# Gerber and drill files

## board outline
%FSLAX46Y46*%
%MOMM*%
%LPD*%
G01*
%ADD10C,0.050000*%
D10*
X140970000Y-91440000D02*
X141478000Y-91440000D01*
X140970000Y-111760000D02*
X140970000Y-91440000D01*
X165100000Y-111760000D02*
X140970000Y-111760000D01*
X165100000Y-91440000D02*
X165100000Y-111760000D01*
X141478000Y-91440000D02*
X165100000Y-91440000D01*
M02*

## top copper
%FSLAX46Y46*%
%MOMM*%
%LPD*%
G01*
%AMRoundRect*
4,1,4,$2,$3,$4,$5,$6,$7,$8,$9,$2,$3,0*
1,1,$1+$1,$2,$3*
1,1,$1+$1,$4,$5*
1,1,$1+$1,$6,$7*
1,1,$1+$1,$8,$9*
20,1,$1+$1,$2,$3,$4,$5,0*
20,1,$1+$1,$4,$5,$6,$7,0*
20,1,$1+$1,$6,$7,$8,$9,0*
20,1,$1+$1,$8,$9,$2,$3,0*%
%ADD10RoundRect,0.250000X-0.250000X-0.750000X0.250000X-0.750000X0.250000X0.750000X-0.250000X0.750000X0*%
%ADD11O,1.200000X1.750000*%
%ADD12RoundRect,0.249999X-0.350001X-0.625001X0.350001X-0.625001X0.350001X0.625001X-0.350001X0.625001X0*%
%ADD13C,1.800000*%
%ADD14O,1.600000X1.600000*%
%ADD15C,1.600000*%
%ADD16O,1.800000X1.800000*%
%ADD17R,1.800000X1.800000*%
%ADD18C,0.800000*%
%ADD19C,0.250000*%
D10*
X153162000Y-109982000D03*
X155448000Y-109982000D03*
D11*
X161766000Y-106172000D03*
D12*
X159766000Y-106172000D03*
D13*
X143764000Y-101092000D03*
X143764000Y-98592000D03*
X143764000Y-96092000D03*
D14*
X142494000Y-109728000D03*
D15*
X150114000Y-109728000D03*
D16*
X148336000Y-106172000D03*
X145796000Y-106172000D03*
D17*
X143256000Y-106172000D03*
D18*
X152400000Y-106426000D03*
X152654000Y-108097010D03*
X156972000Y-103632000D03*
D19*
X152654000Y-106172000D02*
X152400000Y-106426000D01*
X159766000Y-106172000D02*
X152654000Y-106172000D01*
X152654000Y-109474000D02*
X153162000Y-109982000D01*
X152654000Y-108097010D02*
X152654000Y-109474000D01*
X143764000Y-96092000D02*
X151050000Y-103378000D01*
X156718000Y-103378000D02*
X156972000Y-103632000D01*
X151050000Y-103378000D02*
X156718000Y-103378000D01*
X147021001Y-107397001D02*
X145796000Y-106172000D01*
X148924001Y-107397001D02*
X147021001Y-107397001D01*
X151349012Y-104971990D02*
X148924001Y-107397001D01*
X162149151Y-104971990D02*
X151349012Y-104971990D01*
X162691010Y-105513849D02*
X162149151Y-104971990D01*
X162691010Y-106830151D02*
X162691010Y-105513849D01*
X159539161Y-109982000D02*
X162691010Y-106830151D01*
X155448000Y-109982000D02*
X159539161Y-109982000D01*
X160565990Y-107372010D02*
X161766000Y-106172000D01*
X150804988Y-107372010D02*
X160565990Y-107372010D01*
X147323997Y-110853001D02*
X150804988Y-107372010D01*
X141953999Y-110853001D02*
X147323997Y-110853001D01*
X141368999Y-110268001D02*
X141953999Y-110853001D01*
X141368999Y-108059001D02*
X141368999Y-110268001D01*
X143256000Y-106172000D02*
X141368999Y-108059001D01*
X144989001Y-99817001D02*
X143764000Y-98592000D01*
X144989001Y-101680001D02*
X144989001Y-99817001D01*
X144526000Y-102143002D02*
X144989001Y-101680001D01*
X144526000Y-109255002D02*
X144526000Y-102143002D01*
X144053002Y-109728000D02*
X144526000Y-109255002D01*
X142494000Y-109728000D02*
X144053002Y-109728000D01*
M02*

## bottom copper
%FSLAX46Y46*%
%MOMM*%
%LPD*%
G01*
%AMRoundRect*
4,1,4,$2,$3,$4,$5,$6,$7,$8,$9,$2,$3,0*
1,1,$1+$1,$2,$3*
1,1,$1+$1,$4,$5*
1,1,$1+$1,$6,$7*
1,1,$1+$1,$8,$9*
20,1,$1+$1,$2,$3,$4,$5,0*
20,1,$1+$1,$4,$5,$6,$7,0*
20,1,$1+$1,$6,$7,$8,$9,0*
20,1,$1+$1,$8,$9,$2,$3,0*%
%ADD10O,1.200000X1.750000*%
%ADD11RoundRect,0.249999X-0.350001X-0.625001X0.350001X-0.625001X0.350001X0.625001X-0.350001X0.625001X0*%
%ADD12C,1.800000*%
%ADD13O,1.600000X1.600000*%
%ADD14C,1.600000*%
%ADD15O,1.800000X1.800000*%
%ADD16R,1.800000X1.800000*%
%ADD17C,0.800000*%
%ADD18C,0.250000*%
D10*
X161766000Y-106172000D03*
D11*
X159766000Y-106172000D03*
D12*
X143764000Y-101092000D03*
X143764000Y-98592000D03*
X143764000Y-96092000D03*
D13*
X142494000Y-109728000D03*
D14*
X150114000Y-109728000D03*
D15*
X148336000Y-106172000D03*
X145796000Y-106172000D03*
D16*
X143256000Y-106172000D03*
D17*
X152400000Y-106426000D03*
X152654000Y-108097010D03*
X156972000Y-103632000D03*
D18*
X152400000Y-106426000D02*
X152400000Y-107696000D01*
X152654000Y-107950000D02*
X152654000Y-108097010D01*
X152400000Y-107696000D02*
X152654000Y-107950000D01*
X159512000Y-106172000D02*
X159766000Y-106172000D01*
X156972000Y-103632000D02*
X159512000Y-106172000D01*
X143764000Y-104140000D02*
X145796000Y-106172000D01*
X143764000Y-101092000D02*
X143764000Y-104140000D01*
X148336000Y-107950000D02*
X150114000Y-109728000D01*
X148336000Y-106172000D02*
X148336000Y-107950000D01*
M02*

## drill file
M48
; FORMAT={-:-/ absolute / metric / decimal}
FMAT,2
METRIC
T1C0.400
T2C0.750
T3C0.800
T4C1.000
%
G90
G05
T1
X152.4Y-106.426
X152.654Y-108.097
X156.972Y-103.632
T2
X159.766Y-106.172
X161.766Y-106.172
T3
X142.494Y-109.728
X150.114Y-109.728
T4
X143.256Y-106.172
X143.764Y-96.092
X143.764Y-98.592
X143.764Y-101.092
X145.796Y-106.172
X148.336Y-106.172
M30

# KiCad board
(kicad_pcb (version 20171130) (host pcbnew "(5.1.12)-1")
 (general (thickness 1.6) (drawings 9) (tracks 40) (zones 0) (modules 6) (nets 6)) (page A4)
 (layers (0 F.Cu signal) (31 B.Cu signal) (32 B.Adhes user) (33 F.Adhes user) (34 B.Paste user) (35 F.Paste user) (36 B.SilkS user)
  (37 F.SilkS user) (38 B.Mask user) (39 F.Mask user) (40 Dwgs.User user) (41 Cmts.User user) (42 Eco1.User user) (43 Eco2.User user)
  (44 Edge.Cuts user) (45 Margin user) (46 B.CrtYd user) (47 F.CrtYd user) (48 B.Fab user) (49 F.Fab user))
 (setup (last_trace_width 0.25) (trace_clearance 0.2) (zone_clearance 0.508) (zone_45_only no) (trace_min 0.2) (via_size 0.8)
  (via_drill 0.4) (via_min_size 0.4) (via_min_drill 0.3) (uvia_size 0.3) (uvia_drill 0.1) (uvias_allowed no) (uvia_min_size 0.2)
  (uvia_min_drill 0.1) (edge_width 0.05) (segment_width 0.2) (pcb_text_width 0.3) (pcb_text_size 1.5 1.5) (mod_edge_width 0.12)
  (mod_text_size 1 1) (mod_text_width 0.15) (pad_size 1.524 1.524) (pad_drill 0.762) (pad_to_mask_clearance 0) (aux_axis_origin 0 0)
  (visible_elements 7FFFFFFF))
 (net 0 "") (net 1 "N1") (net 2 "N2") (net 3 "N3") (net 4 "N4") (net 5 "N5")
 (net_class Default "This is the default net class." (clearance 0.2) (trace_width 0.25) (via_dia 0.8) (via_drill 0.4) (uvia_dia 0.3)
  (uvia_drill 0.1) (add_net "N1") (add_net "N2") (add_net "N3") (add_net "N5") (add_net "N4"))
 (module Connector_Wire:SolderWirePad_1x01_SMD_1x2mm (layer F.Cu) (at 153.162 109.982)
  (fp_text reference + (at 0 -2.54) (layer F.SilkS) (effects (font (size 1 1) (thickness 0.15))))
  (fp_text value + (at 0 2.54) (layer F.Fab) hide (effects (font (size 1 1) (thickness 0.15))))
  (pad 1 smd roundrect (at 0 0) (size 1 2) (layers F.Cu F.Paste F.Mask) (roundrect_rratio 0.25) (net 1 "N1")))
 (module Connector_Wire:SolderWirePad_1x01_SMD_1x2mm (layer F.Cu) (at 155.448 109.982)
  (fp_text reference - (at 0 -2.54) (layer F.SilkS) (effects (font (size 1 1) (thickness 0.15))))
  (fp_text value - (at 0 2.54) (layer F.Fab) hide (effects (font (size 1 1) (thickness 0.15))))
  (pad 1 smd roundrect (at 0 0) (size 1 2) (layers F.Cu F.Paste F.Mask) (roundrect_rratio 0.25) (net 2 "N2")))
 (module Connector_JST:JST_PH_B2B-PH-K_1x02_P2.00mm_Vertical (layer F.Cu) (at 159.766 106.172)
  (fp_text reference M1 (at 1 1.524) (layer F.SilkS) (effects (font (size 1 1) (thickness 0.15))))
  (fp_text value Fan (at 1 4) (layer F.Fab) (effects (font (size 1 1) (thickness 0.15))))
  (pad 2 thru_hole oval (at 2 0) (size 1.2 1.75) (drill 0.75) (layers *.Cu *.Mask) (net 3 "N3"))
  (pad 1 thru_hole roundrect (at 0 0) (size 1.2 1.75) (drill 0.75) (layers *.Cu *.Mask) (roundrect_rratio 0.2083325) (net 1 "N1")))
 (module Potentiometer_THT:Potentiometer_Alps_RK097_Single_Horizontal (layer F.Cu) (at 143.764 101.092)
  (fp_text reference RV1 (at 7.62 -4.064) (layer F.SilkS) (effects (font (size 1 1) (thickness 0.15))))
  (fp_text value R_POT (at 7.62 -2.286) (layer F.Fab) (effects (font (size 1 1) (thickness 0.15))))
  (pad 1 thru_hole circle (at 0 0) (size 1.8 1.8) (drill 1) (layers *.Cu *.Mask) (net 2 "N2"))
  (pad 2 thru_hole circle (at 0 -2.5) (size 1.8 1.8) (drill 1) (layers *.Cu *.Mask) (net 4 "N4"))
  (pad 3 thru_hole circle (at 0 -5) (size 1.8 1.8) (drill 1) (layers *.Cu *.Mask) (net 1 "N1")))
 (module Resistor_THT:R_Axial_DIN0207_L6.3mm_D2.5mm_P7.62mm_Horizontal (layer F.Cu) (at 150.114 109.728 180)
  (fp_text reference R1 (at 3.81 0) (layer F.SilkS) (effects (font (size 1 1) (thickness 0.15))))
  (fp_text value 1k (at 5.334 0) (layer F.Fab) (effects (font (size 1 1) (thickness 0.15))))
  (pad 2 thru_hole oval (at 7.62 0 180) (size 1.6 1.6) (drill 0.8) (layers *.Cu *.Mask) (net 4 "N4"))
  (pad 1 thru_hole circle (at 0 0 180) (size 1.6 1.6) (drill 0.8) (layers *.Cu *.Mask) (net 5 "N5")))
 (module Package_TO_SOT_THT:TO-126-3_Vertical (layer F.Cu) (at 143.256 106.172)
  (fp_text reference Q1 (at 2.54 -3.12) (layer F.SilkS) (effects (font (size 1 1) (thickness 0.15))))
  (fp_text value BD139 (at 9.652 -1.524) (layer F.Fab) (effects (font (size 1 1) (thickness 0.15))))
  (pad 3 thru_hole oval (at 5.08 0) (size 1.8 1.8) (drill 1) (layers *.Cu *.Mask) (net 5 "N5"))
  (pad 2 thru_hole oval (at 2.54 0) (size 1.8 1.8) (drill 1) (layers *.Cu *.Mask) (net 2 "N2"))
  (pad 1 thru_hole rect (at 0 0) (size 1.8 1.8) (drill 1) (layers *.Cu *.Mask) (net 3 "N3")))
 (gr_line (start 140.97 91.44) (end 141.478 91.44) (layer Edge.Cuts) (width 0.05))
 (gr_line (start 140.97 111.76) (end 140.97 91.44) (layer Edge.Cuts) (width 0.05))
 (gr_line (start 165.1 111.76) (end 140.97 111.76) (layer Edge.Cuts) (width 0.05))
 (gr_line (start 165.1 91.44) (end 165.1 111.76) (layer Edge.Cuts) (width 0.05))
 (gr_line (start 141.478 91.44) (end 165.1 91.44) (layer Edge.Cuts) (width 0.05))
 (via (at 152.4 106.426) (size 0.8) (drill 0.4) (layers F.Cu B.Cu) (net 1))
 (segment (start 152.654 106.172) (end 152.4 106.426) (width 0.25) (layer F.Cu) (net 1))
 (segment (start 159.766 106.172) (end 152.654 106.172) (width 0.25) (layer F.Cu) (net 1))
 (segment (start 152.4 106.426) (end 152.4 107.696) (width 0.25) (layer B.Cu) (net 1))
 (via (at 152.654 108.09701) (size 0.8) (drill 0.4) (layers F.Cu B.Cu) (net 1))
 (segment (start 152.654 107.95) (end 152.654 108.09701) (width 0.25) (layer B.Cu) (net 1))
 (segment (start 152.4 107.696) (end 152.654 107.95) (width 0.25) (layer B.Cu) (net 1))
 (segment (start 152.654 109.474) (end 153.162 109.982) (width 0.25) (layer F.Cu) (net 1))
 (segment (start 152.654 108.09701) (end 152.654 109.474) (width 0.25) (layer F.Cu) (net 1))
 (segment (start 143.764 96.092) (end 151.05 103.378) (width 0.25) (layer F.Cu) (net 1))
 (via (at 156.972 103.632) (size 0.8) (drill 0.4) (layers F.Cu B.Cu) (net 1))
 (segment (start 156.718 103.378) (end 156.972 103.632) (width 0.25) (layer F.Cu) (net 1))
 (segment (start 151.05 103.378) (end 156.718 103.378) (width 0.25) (layer F.Cu) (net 1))
 (segment (start 159.512 106.172) (end 159.766 106.172) (width 0.25) (layer B.Cu) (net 1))
 (segment (start 156.972 103.632) (end 159.512 106.172) (width 0.25) (layer B.Cu) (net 1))
 (segment (start 147.021001 107.397001) (end 145.796 106.172) (width 0.25) (layer F.Cu) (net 2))
 (segment (start 148.924001 107.397001) (end 147.021001 107.397001) (width 0.25) (layer F.Cu) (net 2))
 (segment (start 151.349012 104.97199) (end 148.924001 107.397001) (width 0.25) (layer F.Cu) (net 2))
 (segment (start 162.149151 104.97199) (end 151.349012 104.97199) (width 0.25) (layer F.Cu) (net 2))
 (segment (start 162.69101 105.513849) (end 162.149151 104.97199) (width 0.25) (layer F.Cu) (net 2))
 (segment (start 162.69101 106.830151) (end 162.69101 105.513849) (width 0.25) (layer F.Cu) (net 2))
 (segment (start 159.539161 109.982) (end 162.69101 106.830151) (width 0.25) (layer F.Cu) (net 2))
 (segment (start 155.448 109.982) (end 159.539161 109.982) (width 0.25) (layer F.Cu) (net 2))
 (segment (start 143.764 104.14) (end 145.796 106.172) (width 0.25) (layer B.Cu) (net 2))
 (segment (start 143.764 101.092) (end 143.764 104.14) (width 0.25) (layer B.Cu) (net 2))
 (segment (start 160.56599 107.37201) (end 161.766 106.172) (width 0.25) (layer F.Cu) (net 3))
 (segment (start 150.804988 107.37201) (end 160.56599 107.37201) (width 0.25) (layer F.Cu) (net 3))
 (segment (start 147.323997 110.853001) (end 150.804988 107.37201) (width 0.25) (layer F.Cu) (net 3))
 (segment (start 141.953999 110.853001) (end 147.323997 110.853001) (width 0.25) (layer F.Cu) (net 3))
 (segment (start 141.368999 110.268001) (end 141.953999 110.853001) (width 0.25) (layer F.Cu) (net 3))
 (segment (start 141.368999 108.059001) (end 141.368999 110.268001) (width 0.25) (layer F.Cu) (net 3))
 (segment (start 143.256 106.172) (end 141.368999 108.059001) (width 0.25) (layer F.Cu) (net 3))
 (segment (start 148.336 107.95) (end 150.114 109.728) (width 0.25) (layer B.Cu) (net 5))
 (segment (start 148.336 106.172) (end 148.336 107.95) (width 0.25) (layer B.Cu) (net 5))
 (segment (start 144.989001 99.817001) (end 143.764 98.592) (width 0.25) (layer F.Cu) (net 4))
 (segment (start 144.989001 101.680001) (end 144.989001 99.817001) (width 0.25) (layer F.Cu) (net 4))
 (segment (start 144.526 102.143002) (end 144.989001 101.680001) (width 0.25) (layer F.Cu) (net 4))
 (segment (start 144.526 109.255002) (end 144.526 102.143002) (width 0.25) (layer F.Cu) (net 4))
 (segment (start 144.053002 109.728) (end 144.526 109.255002) (width 0.25) (layer F.Cu) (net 4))
 (segment (start 142.494 109.728) (end 144.053002 109.728) (width 0.25) (layer F.Cu) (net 4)))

